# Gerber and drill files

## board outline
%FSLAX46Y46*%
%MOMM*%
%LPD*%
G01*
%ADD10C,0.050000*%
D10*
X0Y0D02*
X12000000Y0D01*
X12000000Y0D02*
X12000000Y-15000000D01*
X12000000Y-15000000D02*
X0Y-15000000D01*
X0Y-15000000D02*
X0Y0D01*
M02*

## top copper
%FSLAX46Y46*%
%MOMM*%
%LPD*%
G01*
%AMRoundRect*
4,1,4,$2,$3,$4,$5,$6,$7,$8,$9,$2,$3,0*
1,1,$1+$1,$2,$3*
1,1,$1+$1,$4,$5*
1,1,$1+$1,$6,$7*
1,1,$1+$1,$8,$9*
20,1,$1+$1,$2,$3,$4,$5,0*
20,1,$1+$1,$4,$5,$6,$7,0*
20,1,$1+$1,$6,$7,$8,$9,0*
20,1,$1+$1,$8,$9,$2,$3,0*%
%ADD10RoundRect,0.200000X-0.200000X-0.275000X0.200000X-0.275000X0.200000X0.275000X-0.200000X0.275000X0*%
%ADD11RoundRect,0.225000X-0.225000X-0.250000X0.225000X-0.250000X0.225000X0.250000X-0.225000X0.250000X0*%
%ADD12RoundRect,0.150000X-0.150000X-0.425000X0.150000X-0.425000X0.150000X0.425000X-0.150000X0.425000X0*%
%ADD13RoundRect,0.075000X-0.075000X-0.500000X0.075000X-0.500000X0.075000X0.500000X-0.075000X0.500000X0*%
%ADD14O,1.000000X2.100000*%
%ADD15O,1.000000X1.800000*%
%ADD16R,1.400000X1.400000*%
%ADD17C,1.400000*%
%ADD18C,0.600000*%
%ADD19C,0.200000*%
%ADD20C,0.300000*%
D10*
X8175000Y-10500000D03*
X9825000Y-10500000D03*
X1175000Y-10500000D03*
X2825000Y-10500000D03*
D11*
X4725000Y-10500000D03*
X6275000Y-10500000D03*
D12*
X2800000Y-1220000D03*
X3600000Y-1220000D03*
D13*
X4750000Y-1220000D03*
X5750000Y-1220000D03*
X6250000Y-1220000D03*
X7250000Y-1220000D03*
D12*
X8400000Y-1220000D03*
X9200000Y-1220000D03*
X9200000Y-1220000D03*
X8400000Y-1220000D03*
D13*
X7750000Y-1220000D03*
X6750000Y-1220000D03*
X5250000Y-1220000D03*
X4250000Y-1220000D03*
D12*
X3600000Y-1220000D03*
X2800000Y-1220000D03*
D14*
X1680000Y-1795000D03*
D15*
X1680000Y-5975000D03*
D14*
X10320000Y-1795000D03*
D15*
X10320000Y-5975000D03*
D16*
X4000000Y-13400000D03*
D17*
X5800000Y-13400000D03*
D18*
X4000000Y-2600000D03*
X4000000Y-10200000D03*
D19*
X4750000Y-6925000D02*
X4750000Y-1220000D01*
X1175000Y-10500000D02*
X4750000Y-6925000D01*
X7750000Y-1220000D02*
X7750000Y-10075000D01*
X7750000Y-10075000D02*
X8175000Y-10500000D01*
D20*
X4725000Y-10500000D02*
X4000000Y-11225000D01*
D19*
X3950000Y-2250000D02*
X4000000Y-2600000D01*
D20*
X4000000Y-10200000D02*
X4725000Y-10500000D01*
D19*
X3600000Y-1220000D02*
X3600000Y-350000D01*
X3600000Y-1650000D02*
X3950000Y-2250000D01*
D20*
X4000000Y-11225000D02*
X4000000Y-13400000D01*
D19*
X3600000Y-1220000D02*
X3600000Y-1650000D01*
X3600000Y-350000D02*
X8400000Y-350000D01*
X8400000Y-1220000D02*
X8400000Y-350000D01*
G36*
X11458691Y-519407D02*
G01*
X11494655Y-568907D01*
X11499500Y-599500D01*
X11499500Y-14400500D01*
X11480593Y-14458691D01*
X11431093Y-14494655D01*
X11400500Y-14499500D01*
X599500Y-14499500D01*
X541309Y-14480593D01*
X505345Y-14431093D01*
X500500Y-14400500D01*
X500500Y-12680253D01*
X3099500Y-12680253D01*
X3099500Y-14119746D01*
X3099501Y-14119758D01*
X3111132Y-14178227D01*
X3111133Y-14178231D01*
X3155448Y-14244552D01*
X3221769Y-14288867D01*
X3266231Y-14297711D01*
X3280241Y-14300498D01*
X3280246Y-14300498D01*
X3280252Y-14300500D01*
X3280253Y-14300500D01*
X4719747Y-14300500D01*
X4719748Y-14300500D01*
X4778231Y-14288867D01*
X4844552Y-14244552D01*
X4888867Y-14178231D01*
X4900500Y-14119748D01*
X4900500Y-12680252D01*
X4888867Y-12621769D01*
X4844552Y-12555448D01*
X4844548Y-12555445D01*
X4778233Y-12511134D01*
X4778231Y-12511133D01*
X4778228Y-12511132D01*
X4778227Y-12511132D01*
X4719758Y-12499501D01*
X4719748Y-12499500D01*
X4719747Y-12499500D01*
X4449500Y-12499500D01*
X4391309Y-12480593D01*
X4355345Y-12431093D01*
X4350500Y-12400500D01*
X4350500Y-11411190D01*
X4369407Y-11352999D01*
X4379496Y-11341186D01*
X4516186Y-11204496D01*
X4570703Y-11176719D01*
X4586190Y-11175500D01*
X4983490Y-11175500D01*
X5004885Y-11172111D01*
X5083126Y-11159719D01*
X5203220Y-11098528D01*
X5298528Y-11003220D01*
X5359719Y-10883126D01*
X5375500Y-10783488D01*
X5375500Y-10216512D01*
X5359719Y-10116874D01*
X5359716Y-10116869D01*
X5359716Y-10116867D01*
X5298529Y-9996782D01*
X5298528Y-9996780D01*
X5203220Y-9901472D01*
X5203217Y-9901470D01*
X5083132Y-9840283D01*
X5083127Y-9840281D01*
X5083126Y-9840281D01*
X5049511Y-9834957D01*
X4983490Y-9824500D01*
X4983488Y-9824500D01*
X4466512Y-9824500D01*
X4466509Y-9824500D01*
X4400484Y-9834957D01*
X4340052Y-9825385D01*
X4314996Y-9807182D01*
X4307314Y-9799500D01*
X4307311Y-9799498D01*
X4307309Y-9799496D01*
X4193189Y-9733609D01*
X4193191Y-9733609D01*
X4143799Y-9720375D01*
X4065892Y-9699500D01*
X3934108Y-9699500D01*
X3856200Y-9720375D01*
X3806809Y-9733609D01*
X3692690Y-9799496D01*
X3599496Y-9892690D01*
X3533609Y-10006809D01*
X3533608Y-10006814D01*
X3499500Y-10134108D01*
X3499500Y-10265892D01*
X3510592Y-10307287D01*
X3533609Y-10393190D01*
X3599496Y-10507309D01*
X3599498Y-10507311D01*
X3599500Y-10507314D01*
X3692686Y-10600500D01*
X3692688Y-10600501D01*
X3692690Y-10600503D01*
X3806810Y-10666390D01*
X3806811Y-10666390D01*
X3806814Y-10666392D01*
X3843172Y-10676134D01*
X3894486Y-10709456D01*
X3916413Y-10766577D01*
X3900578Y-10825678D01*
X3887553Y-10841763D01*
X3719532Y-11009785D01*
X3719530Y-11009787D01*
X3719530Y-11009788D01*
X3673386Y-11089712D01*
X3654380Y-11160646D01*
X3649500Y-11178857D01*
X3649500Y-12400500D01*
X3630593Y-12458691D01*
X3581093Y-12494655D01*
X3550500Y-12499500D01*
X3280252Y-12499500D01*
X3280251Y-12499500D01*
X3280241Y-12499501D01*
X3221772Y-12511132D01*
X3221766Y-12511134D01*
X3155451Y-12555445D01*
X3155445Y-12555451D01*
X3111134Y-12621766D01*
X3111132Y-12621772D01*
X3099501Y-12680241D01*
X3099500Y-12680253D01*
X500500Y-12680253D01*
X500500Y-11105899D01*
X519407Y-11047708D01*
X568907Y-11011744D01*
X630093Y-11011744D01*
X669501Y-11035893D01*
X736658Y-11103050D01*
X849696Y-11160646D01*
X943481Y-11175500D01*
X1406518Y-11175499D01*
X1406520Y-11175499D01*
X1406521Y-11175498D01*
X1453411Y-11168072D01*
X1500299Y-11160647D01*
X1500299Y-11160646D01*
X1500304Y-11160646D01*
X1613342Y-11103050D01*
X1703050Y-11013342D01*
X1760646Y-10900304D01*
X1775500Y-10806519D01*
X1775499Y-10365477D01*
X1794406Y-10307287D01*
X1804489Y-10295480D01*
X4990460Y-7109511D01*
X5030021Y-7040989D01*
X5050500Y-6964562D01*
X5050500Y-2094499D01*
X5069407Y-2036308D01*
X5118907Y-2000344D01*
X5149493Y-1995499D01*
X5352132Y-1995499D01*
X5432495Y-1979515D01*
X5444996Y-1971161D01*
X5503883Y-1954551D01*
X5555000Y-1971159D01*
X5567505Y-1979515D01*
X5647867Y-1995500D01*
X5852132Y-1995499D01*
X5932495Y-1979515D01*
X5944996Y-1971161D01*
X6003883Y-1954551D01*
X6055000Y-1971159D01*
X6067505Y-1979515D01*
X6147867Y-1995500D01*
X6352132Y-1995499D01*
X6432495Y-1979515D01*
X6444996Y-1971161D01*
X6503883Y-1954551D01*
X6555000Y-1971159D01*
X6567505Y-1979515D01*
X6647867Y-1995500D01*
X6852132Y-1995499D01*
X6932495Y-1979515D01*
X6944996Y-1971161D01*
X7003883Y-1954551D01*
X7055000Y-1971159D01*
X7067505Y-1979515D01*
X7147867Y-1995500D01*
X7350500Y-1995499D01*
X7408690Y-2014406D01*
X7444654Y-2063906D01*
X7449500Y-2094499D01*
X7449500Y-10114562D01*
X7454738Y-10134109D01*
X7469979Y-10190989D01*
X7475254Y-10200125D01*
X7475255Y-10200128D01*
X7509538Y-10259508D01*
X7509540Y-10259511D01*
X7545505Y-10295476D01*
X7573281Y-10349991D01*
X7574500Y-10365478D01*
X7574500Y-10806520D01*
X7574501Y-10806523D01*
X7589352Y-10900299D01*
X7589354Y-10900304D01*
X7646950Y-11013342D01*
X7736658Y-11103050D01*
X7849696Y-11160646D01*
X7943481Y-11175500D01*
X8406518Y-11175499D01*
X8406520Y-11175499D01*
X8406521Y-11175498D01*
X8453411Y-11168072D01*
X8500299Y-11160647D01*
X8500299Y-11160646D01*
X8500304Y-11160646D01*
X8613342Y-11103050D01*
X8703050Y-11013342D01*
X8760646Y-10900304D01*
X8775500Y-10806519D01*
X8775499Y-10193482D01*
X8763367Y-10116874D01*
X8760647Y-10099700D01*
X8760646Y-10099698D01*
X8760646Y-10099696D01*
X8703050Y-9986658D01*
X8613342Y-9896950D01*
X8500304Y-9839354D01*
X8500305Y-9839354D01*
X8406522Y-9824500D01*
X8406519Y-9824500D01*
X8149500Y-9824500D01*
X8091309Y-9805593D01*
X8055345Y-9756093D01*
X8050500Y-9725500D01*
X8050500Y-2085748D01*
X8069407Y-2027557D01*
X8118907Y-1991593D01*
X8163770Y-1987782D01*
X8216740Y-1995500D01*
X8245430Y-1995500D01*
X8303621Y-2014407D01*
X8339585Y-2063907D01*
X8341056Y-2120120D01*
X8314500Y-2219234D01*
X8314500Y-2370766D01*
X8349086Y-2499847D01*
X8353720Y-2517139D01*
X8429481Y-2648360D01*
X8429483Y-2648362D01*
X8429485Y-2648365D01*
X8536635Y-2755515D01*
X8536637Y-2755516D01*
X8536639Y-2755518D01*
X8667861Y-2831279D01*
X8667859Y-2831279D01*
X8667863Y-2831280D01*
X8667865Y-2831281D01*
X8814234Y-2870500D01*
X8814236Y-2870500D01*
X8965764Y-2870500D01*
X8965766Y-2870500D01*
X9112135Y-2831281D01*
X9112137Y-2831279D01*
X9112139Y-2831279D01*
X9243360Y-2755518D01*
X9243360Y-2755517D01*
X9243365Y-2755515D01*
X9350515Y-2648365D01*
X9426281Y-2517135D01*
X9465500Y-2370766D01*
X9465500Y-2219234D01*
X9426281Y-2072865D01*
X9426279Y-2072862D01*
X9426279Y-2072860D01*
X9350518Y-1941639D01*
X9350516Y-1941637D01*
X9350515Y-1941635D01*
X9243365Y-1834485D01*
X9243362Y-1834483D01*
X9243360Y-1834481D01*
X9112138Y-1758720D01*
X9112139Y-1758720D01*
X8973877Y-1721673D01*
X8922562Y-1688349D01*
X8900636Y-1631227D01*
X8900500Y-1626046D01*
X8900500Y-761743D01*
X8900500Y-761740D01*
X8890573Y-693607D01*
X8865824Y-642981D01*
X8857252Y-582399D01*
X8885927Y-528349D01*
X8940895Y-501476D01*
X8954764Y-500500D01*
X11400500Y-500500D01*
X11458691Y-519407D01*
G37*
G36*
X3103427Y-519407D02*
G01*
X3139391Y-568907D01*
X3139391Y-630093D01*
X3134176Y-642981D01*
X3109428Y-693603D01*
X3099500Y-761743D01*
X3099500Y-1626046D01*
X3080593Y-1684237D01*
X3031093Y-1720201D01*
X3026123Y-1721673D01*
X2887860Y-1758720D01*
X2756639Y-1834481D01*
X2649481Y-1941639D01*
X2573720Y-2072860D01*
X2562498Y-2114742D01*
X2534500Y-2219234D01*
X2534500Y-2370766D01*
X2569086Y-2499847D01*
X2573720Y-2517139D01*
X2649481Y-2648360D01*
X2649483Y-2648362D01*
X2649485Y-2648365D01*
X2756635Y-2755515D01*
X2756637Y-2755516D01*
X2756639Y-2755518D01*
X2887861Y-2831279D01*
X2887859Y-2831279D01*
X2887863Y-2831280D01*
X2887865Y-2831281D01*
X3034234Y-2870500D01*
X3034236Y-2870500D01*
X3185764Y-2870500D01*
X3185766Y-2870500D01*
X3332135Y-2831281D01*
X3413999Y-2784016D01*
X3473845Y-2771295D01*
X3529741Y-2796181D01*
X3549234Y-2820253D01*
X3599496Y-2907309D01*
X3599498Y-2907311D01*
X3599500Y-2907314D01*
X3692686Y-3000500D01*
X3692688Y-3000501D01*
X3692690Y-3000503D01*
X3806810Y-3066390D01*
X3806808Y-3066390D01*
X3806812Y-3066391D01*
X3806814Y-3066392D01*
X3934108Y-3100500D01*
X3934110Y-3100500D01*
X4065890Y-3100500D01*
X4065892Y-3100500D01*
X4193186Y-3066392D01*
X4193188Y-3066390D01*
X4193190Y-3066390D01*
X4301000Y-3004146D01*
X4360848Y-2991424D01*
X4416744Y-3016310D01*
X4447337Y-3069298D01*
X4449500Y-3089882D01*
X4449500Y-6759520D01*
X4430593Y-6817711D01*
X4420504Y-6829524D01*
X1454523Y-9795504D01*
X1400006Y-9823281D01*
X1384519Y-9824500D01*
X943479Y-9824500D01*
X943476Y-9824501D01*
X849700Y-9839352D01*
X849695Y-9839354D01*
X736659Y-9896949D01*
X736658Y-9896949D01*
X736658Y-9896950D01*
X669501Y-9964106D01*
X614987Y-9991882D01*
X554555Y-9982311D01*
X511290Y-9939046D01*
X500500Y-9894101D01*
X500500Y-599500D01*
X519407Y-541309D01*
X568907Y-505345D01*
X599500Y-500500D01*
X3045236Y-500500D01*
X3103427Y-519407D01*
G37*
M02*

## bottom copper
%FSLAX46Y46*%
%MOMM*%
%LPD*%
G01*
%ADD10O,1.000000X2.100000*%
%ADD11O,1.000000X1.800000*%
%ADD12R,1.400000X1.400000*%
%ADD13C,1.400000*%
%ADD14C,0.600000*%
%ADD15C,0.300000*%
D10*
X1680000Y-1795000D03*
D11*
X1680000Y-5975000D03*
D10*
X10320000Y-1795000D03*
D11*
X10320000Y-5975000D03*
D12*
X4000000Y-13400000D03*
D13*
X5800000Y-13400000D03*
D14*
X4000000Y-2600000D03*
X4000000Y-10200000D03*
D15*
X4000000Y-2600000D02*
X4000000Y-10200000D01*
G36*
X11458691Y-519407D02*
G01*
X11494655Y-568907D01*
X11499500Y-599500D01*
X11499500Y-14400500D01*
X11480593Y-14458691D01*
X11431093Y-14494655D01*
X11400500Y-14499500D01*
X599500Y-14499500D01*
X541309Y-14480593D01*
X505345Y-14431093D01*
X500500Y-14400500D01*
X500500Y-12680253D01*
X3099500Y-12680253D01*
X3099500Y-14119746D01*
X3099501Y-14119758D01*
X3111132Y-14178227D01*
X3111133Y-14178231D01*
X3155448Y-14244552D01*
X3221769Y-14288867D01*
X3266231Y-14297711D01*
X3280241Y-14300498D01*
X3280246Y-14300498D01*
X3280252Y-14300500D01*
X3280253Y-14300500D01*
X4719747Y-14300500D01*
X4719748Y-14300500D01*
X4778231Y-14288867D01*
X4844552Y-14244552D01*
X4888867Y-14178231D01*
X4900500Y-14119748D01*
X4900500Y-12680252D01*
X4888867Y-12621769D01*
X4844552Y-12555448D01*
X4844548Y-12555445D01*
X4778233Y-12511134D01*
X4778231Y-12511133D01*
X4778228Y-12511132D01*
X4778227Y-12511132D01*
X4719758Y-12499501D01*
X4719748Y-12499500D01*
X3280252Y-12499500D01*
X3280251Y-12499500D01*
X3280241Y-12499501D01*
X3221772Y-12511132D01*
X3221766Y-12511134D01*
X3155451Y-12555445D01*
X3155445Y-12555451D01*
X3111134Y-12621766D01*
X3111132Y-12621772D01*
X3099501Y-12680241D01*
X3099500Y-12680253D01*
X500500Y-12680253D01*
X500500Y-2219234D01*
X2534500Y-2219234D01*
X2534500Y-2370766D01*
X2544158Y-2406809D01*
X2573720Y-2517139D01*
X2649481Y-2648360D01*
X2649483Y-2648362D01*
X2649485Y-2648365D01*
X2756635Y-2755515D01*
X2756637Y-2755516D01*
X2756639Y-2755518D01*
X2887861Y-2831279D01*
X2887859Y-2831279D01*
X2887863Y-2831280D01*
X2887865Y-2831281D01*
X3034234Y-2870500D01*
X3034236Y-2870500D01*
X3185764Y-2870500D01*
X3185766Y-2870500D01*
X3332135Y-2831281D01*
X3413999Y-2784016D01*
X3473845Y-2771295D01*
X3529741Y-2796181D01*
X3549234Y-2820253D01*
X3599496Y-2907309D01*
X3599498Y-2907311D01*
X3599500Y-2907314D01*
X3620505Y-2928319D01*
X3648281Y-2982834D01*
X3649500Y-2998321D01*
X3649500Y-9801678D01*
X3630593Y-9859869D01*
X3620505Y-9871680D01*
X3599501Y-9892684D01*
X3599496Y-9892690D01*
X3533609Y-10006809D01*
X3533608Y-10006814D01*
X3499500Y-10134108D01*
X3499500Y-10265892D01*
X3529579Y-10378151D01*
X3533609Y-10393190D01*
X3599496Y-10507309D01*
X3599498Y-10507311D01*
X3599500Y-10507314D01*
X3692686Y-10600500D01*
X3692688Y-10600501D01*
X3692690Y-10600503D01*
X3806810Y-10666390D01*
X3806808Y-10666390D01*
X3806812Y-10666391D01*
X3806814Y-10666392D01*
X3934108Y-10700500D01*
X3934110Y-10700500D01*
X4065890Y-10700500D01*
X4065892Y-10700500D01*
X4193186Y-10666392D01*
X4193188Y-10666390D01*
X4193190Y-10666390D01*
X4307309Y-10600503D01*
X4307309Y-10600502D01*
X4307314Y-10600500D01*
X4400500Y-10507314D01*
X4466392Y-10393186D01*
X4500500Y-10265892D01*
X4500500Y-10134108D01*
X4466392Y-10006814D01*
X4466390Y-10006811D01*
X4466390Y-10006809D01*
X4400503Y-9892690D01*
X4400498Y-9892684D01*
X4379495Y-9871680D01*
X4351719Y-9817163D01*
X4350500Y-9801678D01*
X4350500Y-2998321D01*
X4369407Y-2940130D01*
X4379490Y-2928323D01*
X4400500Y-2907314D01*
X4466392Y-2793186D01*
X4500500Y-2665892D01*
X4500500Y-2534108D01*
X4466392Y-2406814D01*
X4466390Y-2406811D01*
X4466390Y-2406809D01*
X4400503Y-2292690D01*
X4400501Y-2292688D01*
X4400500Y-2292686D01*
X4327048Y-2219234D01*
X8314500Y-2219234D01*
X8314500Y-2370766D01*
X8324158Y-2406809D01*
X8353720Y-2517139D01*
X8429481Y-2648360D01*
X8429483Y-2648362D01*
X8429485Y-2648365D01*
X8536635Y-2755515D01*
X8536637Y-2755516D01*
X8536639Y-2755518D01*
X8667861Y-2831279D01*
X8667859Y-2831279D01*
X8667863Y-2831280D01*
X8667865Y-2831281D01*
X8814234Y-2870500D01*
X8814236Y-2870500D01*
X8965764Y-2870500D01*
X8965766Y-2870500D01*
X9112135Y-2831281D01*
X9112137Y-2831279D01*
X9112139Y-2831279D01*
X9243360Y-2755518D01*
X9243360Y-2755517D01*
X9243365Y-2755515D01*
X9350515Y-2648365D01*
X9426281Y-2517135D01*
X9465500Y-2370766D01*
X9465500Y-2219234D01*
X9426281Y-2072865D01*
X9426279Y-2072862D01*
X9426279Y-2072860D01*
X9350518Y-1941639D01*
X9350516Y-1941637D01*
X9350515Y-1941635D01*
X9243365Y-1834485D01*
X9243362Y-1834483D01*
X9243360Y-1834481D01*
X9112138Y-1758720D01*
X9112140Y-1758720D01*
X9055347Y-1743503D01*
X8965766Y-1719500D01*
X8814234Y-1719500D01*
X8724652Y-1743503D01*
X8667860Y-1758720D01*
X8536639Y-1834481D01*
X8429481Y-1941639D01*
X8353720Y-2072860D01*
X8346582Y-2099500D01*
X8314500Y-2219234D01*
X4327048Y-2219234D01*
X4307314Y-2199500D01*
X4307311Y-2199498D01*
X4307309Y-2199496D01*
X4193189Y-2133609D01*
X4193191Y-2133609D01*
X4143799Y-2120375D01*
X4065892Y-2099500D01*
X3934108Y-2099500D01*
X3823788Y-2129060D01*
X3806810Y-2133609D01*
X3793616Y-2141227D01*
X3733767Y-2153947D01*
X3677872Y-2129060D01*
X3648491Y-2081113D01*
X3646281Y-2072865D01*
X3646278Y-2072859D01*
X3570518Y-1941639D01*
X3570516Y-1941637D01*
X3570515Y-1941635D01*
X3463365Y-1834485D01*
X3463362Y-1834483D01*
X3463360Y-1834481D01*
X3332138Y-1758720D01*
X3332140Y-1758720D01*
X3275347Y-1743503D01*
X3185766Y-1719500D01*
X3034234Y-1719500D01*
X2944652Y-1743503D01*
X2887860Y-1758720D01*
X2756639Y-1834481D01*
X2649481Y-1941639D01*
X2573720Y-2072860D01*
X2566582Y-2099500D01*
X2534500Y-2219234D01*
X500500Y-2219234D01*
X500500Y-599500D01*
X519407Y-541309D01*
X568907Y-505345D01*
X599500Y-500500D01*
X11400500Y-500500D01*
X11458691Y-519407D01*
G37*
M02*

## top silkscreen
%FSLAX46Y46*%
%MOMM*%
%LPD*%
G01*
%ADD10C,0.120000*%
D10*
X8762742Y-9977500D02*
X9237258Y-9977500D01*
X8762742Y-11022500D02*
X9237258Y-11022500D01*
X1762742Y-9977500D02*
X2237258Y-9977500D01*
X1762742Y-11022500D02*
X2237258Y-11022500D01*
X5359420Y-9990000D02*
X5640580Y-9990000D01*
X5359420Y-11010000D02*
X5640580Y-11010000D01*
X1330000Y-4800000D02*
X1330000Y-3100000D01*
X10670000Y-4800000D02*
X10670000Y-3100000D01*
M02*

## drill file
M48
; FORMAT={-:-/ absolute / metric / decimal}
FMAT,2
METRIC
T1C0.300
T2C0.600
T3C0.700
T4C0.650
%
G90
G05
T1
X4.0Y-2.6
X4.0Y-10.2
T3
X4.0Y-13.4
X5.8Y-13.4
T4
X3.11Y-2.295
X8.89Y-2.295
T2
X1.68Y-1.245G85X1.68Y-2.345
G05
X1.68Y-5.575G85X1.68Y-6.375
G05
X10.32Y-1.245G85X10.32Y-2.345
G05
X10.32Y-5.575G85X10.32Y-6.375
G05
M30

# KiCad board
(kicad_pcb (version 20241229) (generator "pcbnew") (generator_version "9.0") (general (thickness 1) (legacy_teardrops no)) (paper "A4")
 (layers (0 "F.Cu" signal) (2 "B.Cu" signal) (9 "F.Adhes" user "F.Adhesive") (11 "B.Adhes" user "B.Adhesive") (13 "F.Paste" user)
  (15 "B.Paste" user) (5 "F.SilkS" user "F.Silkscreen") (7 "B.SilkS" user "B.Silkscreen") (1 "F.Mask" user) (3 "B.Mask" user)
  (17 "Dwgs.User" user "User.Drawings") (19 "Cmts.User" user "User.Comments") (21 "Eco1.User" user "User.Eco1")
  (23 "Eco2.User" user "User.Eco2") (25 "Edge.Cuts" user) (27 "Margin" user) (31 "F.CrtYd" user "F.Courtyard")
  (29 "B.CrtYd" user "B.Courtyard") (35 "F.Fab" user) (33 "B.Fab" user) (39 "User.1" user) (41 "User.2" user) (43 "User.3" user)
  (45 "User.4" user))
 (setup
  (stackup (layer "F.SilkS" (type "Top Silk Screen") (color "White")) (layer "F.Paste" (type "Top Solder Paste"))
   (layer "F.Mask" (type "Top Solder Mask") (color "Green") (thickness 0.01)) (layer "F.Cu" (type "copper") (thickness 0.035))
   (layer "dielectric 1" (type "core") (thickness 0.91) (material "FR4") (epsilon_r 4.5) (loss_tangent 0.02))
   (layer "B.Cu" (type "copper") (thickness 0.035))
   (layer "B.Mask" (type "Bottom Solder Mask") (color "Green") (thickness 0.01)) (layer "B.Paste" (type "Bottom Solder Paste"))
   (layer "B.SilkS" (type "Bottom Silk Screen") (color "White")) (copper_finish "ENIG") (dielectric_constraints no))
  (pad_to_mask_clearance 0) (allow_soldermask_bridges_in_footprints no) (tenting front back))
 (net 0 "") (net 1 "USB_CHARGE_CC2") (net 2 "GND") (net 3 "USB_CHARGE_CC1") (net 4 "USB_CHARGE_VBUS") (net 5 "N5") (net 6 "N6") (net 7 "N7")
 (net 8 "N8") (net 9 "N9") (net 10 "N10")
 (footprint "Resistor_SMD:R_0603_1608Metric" (layer "F.Cu") (at 9 10.5)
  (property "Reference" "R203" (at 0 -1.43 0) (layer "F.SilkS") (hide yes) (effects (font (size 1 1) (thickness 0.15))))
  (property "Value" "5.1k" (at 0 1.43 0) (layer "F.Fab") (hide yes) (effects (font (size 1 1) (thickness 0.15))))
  (fp_line (start -0.237258 -0.5225) (end 0.237258 -0.5225) (stroke (width 0.12) (type solid)) (layer "F.SilkS"))
  (fp_line (start -0.237258 0.5225) (end 0.237258 0.5225) (stroke (width 0.12) (type solid)) (layer "F.SilkS"))
  (pad "1" smd roundrect (at -0.825 0) (size 0.8 0.95) (layers "F.Cu" "F.Mask" "F.Paste") (roundrect_rratio 0.25) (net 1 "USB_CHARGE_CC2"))
  (pad "2" smd roundrect (at 0.825 0) (size 0.8 0.95) (layers "F.Cu" "F.Mask" "F.Paste") (roundrect_rratio 0.25) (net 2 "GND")
   (zone_connect 2)))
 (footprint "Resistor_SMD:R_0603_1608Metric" (layer "F.Cu") (at 2 10.5)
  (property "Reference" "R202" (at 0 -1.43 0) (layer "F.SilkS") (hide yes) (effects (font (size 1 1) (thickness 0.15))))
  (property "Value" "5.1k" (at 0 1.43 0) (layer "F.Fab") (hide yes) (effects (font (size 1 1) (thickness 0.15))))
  (fp_line (start -0.237258 -0.5225) (end 0.237258 -0.5225) (stroke (width 0.12) (type solid)) (layer "F.SilkS"))
  (fp_line (start -0.237258 0.5225) (end 0.237258 0.5225) (stroke (width 0.12) (type solid)) (layer "F.SilkS"))
  (pad "1" smd roundrect (at -0.825 0) (size 0.8 0.95) (layers "F.Cu" "F.Mask" "F.Paste") (roundrect_rratio 0.25) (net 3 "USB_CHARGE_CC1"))
  (pad "2" smd roundrect (at 0.825 0) (size 0.8 0.95) (layers "F.Cu" "F.Mask" "F.Paste") (roundrect_rratio 0.25) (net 2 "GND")
   (zone_connect 2)))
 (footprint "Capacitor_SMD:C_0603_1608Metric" (layer "F.Cu") (at 5.5 10.5)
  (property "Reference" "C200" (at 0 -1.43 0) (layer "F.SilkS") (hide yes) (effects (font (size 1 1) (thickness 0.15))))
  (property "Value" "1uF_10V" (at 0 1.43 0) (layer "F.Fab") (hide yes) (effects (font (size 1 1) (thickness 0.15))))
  (fp_line (start -0.14058 -0.51) (end 0.14058 -0.51) (stroke (width 0.12) (type solid)) (layer "F.SilkS"))
  (fp_line (start -0.14058 0.51) (end 0.14058 0.51) (stroke (width 0.12) (type solid)) (layer "F.SilkS"))
  (pad "1" smd roundrect (at -0.775 0) (size 0.9 0.95) (layers "F.Cu" "F.Mask" "F.Paste") (roundrect_rratio 0.25) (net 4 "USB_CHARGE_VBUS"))
  (pad "2" smd roundrect (at 0.775 0) (size 0.9 0.95) (layers "F.Cu" "F.Mask" "F.Paste") (roundrect_rratio 0.25) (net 2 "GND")
   (zone_connect 2)))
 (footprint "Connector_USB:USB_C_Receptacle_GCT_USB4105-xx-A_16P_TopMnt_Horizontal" (layer "F.Cu") (at 6 4.9)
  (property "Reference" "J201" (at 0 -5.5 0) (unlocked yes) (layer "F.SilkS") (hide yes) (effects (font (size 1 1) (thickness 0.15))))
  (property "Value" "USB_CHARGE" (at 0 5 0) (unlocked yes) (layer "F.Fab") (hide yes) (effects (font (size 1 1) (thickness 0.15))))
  (fp_line (start -4.67 -0.1) (end -4.67 -1.8) (stroke (width 0.12) (type solid)) (layer "F.SilkS"))
  (fp_line (start 4.67 -0.1) (end 4.67 -1.8) (stroke (width 0.12) (type solid)) (layer "F.SilkS"))
  (pad "" np_thru_hole circle (at -2.89 -2.605) (size 0.65 0.65) (drill 0.65) (layers "*.Cu" "*.Mask"))
  (pad "" np_thru_hole circle (at 2.89 -2.605) (size 0.65 0.65) (drill 0.65) (layers "*.Cu" "*.Mask"))
  (pad "A1" smd roundrect (at -3.2 -3.68) (size 0.6 1.15) (layers "F.Cu" "F.Mask" "F.Paste") (roundrect_rratio 0.25) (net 2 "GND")
   (zone_connect 2))
  (pad "A4" smd roundrect (at -2.4 -3.68) (size 0.6 1.15) (layers "F.Cu" "F.Mask" "F.Paste") (roundrect_rratio 0.25)
   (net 4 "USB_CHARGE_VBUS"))
  (pad "A5" smd roundrect (at -1.25 -3.68) (size 0.3 1.15) (layers "F.Cu" "F.Mask" "F.Paste") (roundrect_rratio 0.25)
   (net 3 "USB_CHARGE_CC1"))
  (pad "A6" smd roundrect (at -0.25 -3.68) (size 0.3 1.15) (layers "F.Cu" "F.Mask" "F.Paste") (roundrect_rratio 0.25) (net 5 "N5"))
  (pad "A7" smd roundrect (at 0.25 -3.68) (size 0.3 1.15) (layers "F.Cu" "F.Mask" "F.Paste") (roundrect_rratio 0.25) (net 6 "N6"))
  (pad "A8" smd roundrect (at 1.25 -3.68) (size 0.3 1.15) (layers "F.Cu" "F.Mask" "F.Paste") (roundrect_rratio 0.25) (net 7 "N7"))
  (pad "A9" smd roundrect (at 2.4 -3.68) (size 0.6 1.15) (layers "F.Cu" "F.Mask" "F.Paste") (roundrect_rratio 0.25)
   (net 4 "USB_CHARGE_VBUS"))
  (pad "A12" smd roundrect (at 3.2 -3.68) (size 0.6 1.15) (layers "F.Cu" "F.Mask" "F.Paste") (roundrect_rratio 0.25) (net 2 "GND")
   (zone_connect 2))
  (pad "B1" smd roundrect (at 3.2 -3.68) (size 0.6 1.15) (layers "F.Cu" "F.Mask" "F.Paste") (roundrect_rratio 0.25) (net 2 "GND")
   (zone_connect 2))
  (pad "B4" smd roundrect (at 2.4 -3.68) (size 0.6 1.15) (layers "F.Cu" "F.Mask" "F.Paste") (roundrect_rratio 0.25)
   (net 4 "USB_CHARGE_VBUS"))
  (pad "B5" smd roundrect (at 1.75 -3.68) (size 0.3 1.15) (layers "F.Cu" "F.Mask" "F.Paste") (roundrect_rratio 0.25)
   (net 1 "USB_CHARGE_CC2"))
  (pad "B6" smd roundrect (at 0.75 -3.68) (size 0.3 1.15) (layers "F.Cu" "F.Mask" "F.Paste") (roundrect_rratio 0.25) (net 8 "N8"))
  (pad "B7" smd roundrect (at -0.75 -3.68) (size 0.3 1.15) (layers "F.Cu" "F.Mask" "F.Paste") (roundrect_rratio 0.25) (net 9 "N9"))
  (pad "B8" smd roundrect (at -1.75 -3.68) (size 0.3 1.15) (layers "F.Cu" "F.Mask" "F.Paste") (roundrect_rratio 0.25) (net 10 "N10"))
  (pad "B9" smd roundrect (at -2.4 -3.68) (size 0.6 1.15) (layers "F.Cu" "F.Mask" "F.Paste") (roundrect_rratio 0.25)
   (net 4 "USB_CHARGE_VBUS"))
  (pad "B12" smd roundrect (at -3.2 -3.68) (size 0.6 1.15) (layers "F.Cu" "F.Mask" "F.Paste") (roundrect_rratio 0.25) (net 2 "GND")
   (zone_connect 2))
  (pad "S1" thru_hole oval (at -4.32 -3.105) (size 1 2.1) (drill oval 0.6 1.7) (layers "*.Cu" "*.Mask" "F.Paste") (remove_unused_layers no)
   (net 2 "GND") (zone_connect 2))
  (pad "S1" thru_hole oval (at -4.32 1.075) (size 1 1.8) (drill oval 0.6 1.4) (layers "*.Cu" "*.Mask" "F.Paste") (remove_unused_layers no)
   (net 2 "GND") (zone_connect 2))
  (pad "S1" thru_hole oval (at 4.32 -3.105) (size 1 2.1) (drill oval 0.6 1.7) (layers "*.Cu" "*.Mask" "F.Paste") (remove_unused_layers no)
   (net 2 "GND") (zone_connect 2))
  (pad "S1" thru_hole oval (at 4.32 1.075) (size 1 1.8) (drill oval 0.6 1.4) (layers "*.Cu" "*.Mask" "F.Paste") (remove_unused_layers no)
   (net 2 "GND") (zone_connect 2)))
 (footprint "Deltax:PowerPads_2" (layer "F.Cu") (at 4 13.4)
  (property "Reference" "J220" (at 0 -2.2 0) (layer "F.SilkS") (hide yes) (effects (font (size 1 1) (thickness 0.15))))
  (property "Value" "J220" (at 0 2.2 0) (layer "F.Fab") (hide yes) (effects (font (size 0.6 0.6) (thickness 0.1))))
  (pad "1" thru_hole rect (at 0 0) (size 1.4 1.4) (drill 0.7) (layers "*.Cu" "*.Mask") (remove_unused_layers no) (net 4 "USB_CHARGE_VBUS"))
  (pad "2" thru_hole circle (at 1.8 0) (size 1.4 1.4) (drill 0.7) (layers "*.Cu" "*.Mask") (remove_unused_layers no) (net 2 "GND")
   (zone_connect 2)))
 (gr_line (start 0 0) (end 12 0) (stroke (width 0.05) (type default)) (layer "Edge.Cuts"))
 (gr_line (start 12 0) (end 12 15) (stroke (width 0.05) (type default)) (layer "Edge.Cuts"))
 (gr_line (start 12 15) (end 0 15) (stroke (width 0.05) (type default)) (layer "Edge.Cuts"))
 (gr_line (start 0 15) (end 0 0) (stroke (width 0.05) (type default)) (layer "Edge.Cuts"))
 (segment (start 4.75 6.925) (end 4.75 1.22) (width 0.2) (layer "F.Cu") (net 3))
 (segment (start 1.175 10.5) (end 4.75 6.925) (width 0.2) (layer "F.Cu") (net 3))
 (segment (start 7.75 1.22) (end 7.75 10.075) (width 0.2) (layer "F.Cu") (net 1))
 (segment (start 7.75 10.075) (end 8.175 10.5) (width 0.2) (layer "F.Cu") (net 1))
 (segment (start 4.725 10.5) (end 4 11.225) (width 0.3) (layer "F.Cu") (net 4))
 (segment (start 3.95 2.25) (end 4 2.6) (width 0.2) (layer "F.Cu") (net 4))
 (segment (start 4 10.2) (end 4.725 10.5) (width 0.3) (layer "F.Cu") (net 4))
 (segment (start 3.6 1.22) (end 3.6 0.35) (width 0.2) (layer "F.Cu") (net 4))
 (segment (start 3.6 1.65) (end 3.95 2.25) (width 0.2) (layer "F.Cu") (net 4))
 (segment (start 4 11.225) (end 4 13.4) (width 0.3) (layer "F.Cu") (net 4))
 (segment (start 3.6 1.22) (end 3.6 1.65) (width 0.2) (layer "F.Cu") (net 4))
 (segment (start 3.6 0.35) (end 8.4 0.35) (width 0.2) (layer "F.Cu") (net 4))
 (segment (start 8.4 1.22) (end 8.4 0.35) (width 0.2) (layer "F.Cu") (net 4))
 (via (at 4 2.6) (size 0.6) (drill 0.3) (layers "F.Cu" "B.Cu") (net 4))
 (via (at 4 10.2) (size 0.6) (drill 0.3) (layers "F.Cu" "B.Cu") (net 4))
 (segment (start 4 2.6) (end 4 10.2) (width 0.3) (layer "B.Cu") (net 4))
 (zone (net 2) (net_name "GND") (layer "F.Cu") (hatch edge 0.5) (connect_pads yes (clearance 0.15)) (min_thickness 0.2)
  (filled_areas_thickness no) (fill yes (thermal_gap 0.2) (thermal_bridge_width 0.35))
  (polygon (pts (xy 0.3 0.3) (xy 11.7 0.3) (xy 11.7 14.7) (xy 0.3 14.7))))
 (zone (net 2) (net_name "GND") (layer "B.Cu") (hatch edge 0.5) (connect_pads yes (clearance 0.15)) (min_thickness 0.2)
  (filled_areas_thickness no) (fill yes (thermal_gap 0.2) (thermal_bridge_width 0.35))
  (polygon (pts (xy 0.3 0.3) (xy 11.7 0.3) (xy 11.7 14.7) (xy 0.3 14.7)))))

